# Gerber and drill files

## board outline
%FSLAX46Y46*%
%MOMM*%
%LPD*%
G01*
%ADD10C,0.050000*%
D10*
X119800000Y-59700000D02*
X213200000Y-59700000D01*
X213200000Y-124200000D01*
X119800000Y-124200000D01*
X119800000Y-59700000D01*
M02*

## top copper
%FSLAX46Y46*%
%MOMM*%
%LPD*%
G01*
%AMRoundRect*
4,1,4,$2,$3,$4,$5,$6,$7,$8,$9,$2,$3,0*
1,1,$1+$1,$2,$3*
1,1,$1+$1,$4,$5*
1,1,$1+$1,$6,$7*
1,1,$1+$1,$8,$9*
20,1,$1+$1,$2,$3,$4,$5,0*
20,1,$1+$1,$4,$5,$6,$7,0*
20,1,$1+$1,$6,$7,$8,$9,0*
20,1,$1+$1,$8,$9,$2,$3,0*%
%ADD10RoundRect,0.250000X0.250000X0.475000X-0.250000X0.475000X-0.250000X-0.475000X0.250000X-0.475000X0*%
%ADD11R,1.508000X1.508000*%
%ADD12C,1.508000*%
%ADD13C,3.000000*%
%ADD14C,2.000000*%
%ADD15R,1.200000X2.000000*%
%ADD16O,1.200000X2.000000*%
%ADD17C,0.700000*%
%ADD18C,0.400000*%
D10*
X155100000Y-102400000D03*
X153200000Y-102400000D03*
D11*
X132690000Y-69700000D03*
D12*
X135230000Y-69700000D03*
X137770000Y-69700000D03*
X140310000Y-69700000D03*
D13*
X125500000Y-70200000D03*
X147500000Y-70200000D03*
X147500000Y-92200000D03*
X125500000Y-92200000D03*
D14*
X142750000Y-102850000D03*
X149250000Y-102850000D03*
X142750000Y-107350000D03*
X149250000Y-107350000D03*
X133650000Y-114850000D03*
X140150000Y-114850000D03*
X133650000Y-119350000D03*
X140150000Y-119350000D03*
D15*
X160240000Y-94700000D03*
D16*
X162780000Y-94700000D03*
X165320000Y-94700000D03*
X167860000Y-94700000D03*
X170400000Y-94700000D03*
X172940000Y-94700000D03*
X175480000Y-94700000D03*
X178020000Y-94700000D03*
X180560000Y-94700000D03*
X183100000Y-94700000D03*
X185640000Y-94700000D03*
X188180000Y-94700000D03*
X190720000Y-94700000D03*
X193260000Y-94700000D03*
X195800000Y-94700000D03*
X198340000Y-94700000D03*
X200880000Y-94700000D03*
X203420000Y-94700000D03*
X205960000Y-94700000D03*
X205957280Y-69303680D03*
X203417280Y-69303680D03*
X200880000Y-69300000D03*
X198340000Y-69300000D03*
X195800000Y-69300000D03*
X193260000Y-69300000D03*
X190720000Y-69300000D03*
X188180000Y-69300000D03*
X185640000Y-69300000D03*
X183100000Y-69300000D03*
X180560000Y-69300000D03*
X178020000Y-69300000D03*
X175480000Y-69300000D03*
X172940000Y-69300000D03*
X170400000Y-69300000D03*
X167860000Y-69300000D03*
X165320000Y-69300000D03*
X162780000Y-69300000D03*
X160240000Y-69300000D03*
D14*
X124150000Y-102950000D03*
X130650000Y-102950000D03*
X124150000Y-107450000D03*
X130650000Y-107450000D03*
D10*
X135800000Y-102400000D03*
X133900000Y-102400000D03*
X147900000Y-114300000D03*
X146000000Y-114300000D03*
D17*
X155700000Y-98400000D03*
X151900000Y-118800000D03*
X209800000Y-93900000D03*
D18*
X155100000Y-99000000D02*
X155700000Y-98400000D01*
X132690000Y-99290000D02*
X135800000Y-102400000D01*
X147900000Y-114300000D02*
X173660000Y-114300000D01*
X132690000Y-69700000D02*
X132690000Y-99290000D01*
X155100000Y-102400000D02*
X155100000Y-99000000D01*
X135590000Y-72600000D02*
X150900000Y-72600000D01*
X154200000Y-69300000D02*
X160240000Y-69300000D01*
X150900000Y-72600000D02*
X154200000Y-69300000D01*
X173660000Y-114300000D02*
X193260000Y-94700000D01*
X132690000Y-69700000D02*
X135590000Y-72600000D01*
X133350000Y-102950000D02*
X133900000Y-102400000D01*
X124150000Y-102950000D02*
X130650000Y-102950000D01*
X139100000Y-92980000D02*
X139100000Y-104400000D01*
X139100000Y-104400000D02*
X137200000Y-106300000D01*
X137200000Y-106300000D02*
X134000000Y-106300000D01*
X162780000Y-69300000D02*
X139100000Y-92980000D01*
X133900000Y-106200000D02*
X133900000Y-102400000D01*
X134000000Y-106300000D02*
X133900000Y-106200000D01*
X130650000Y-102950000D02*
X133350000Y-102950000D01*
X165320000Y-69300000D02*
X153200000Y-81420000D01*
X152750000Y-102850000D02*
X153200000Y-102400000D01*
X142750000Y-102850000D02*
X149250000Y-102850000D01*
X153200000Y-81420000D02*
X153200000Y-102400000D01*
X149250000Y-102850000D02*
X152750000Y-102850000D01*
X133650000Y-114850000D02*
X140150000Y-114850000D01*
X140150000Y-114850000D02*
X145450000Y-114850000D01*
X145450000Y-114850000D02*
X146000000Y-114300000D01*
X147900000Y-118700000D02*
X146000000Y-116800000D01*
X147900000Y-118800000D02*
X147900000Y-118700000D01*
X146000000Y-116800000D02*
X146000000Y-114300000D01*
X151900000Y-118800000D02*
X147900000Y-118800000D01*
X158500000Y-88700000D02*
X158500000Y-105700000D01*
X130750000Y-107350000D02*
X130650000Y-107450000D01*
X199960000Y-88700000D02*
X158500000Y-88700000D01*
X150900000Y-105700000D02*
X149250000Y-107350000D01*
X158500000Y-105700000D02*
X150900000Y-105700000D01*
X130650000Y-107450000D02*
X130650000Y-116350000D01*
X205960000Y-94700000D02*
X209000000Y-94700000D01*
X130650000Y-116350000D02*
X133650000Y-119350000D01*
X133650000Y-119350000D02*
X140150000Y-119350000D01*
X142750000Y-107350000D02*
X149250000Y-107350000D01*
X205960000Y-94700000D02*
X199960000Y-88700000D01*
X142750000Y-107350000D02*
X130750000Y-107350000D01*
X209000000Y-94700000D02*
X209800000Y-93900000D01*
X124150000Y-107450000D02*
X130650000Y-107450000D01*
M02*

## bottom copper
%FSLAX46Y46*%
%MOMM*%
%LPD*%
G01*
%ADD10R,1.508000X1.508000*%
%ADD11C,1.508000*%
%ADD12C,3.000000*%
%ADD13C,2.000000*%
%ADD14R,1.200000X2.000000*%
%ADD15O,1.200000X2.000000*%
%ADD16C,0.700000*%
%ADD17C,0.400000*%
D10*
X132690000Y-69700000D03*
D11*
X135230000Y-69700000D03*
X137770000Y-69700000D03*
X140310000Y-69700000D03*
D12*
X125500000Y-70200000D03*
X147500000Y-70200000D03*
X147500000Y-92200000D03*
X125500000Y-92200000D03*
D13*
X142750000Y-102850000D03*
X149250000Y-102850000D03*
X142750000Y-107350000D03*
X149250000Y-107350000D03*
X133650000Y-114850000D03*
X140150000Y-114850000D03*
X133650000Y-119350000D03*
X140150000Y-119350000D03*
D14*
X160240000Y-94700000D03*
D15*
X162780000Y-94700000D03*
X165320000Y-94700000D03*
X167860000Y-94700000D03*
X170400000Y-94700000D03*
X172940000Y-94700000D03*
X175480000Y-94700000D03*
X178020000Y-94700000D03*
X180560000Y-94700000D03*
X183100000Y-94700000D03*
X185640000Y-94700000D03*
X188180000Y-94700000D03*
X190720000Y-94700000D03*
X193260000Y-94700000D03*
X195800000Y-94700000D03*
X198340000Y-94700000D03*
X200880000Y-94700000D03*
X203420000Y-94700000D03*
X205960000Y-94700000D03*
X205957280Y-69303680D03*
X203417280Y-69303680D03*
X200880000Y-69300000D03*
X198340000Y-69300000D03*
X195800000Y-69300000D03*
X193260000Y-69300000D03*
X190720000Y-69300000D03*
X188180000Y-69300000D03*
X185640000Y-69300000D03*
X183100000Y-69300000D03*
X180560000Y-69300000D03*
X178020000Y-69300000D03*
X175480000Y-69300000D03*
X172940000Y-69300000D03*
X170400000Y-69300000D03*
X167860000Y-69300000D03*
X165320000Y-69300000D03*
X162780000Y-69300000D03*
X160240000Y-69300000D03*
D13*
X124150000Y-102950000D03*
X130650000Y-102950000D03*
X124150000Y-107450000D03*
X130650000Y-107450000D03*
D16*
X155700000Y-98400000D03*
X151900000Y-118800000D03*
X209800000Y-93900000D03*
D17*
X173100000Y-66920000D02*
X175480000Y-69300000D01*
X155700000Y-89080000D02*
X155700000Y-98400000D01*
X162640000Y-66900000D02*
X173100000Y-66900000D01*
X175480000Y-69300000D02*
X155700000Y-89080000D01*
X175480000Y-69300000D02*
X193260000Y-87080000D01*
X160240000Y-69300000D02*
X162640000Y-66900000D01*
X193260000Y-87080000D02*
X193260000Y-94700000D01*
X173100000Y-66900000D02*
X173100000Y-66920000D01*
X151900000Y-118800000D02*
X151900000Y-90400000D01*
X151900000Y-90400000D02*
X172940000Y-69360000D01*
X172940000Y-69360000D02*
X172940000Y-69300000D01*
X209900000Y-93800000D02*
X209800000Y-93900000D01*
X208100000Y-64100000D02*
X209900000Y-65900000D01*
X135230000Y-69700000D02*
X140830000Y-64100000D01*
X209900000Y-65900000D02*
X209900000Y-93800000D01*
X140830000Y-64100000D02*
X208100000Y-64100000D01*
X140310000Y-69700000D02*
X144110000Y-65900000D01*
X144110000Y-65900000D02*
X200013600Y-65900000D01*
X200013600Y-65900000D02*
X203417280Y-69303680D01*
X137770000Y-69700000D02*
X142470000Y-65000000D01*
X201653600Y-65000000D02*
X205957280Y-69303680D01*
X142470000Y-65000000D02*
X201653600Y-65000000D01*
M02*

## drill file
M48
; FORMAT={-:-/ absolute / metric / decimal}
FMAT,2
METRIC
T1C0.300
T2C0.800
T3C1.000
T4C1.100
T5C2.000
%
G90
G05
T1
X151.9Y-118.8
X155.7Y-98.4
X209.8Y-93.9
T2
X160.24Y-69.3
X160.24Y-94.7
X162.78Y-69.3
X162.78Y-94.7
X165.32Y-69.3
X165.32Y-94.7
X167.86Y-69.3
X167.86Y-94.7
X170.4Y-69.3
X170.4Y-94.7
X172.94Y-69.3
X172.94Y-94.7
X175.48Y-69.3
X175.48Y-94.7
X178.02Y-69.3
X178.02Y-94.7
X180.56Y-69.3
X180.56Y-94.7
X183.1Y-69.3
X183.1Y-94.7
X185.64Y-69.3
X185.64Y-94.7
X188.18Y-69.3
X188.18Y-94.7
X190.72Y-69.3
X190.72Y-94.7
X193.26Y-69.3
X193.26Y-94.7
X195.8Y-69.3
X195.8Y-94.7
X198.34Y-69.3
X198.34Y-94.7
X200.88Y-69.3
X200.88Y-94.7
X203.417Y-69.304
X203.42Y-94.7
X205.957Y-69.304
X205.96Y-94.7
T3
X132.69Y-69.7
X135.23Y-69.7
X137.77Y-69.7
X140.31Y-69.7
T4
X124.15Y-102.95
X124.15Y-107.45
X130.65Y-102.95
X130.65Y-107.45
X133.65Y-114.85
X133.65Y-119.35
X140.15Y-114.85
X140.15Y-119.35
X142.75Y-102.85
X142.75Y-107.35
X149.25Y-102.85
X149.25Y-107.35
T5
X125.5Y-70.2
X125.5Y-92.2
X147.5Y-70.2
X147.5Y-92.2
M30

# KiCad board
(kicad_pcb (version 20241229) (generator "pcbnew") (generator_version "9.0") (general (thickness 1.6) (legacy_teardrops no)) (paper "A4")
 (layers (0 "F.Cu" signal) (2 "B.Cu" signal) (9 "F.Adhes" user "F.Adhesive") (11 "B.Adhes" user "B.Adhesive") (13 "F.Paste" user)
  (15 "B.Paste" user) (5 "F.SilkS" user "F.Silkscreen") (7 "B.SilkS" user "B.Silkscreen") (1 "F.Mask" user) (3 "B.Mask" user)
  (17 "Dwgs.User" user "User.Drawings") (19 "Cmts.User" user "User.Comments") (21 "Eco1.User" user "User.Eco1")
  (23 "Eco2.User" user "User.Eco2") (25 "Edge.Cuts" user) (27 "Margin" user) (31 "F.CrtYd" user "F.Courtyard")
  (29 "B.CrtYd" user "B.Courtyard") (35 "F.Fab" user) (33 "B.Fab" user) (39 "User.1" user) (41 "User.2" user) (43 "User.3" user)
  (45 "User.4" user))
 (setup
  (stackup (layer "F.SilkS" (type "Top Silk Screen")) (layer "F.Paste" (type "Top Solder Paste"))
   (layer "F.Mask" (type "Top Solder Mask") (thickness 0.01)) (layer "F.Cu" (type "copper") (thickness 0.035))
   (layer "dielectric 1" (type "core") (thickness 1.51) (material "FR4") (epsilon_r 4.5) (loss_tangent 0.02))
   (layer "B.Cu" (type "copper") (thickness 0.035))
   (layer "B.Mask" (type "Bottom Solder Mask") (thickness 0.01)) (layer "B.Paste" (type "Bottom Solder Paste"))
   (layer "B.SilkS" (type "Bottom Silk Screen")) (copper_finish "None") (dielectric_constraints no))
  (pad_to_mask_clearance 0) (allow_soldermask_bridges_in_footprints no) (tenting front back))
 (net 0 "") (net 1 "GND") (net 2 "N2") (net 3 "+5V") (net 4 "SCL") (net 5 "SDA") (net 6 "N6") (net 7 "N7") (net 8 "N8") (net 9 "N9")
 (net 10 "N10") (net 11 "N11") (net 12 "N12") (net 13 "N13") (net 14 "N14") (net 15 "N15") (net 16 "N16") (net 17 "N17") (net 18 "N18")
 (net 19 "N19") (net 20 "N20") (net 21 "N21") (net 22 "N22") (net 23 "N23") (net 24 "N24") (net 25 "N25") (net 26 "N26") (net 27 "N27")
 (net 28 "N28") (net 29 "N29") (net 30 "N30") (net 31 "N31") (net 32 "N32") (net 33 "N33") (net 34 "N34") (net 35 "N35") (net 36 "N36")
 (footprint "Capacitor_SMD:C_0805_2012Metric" (layer "F.Cu") (at 154.15 102.4 180)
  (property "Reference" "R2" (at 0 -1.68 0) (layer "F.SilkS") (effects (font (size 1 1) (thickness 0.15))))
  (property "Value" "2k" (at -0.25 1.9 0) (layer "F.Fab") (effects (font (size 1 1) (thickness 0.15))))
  (pad "1" smd roundrect (at -0.95 0 180) (size 1 1.45) (layers "F.Cu" "F.Mask" "F.Paste") (roundrect_rratio 0.25) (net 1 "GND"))
  (pad "2" smd roundrect (at 0.95 0 180) (size 1 1.45) (layers "F.Cu" "F.Mask" "F.Paste") (roundrect_rratio 0.25) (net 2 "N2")))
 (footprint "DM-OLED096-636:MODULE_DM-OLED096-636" (layer "F.Cu") (at 136.5 81.2)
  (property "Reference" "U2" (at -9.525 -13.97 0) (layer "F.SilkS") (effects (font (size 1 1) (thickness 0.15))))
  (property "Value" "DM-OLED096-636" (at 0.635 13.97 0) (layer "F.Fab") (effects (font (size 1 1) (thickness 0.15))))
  (pad "1" thru_hole rect (at -3.81 -11.5) (size 1.508 1.508) (drill 1) (layers "*.Cu" "*.Mask") (remove_unused_layers no) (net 1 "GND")
   (solder_mask_margin 0.102))
  (pad "2" thru_hole circle (at -1.27 -11.5) (size 1.508 1.508) (drill 1) (layers "*.Cu" "*.Mask") (remove_unused_layers no) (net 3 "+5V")
   (solder_mask_margin 0.102))
  (pad "3" thru_hole circle (at 1.27 -11.5) (size 1.508 1.508) (drill 1) (layers "*.Cu" "*.Mask") (remove_unused_layers no) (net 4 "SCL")
   (solder_mask_margin 0.102))
  (pad "4" thru_hole circle (at 3.81 -11.5) (size 1.508 1.508) (drill 1) (layers "*.Cu" "*.Mask") (remove_unused_layers no) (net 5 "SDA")
   (solder_mask_margin 0.102))
  (pad "S1" thru_hole circle (at -11 -11) (size 3 3) (drill 2) (layers "*.Cu" "*.Mask") (remove_unused_layers no) (solder_mask_margin 0.102))
  (pad "S2" thru_hole circle (at 11 -11) (size 3 3) (drill 2) (layers "*.Cu" "*.Mask") (remove_unused_layers no) (solder_mask_margin 0.102))
  (pad "S3" thru_hole circle (at 11 11) (size 3 3) (drill 2) (layers "*.Cu" "*.Mask") (remove_unused_layers no) (solder_mask_margin 0.102))
  (pad "S4" thru_hole circle (at -11 11) (size 3 3) (drill 2) (layers "*.Cu" "*.Mask") (remove_unused_layers no) (solder_mask_margin 0.102)))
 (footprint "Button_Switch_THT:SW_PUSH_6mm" (layer "F.Cu") (at 142.75 102.85)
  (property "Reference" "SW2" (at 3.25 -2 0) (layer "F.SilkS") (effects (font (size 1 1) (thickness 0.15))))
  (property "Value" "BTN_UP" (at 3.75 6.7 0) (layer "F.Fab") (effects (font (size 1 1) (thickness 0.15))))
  (pad "1" thru_hole circle (at 0 0 90) (size 2 2) (drill 1.1) (layers "*.Cu" "*.Mask") (remove_unused_layers no) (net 2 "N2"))
  (pad "1" thru_hole circle (at 6.5 0 90) (size 2 2) (drill 1.1) (layers "*.Cu" "*.Mask") (remove_unused_layers no) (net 2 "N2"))
  (pad "2" thru_hole circle (at 0 4.5 90) (size 2 2) (drill 1.1) (layers "*.Cu" "*.Mask") (remove_unused_layers no) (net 3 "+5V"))
  (pad "2" thru_hole circle (at 6.5 4.5 90) (size 2 2) (drill 1.1) (layers "*.Cu" "*.Mask") (remove_unused_layers no) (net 3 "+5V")))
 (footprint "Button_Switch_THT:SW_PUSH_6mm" (layer "F.Cu") (at 133.65 114.85)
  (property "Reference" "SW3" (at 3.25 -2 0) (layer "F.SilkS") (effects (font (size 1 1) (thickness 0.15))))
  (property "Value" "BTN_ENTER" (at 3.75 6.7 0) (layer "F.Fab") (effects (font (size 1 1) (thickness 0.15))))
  (pad "1" thru_hole circle (at 0 0 90) (size 2 2) (drill 1.1) (layers "*.Cu" "*.Mask") (remove_unused_layers no) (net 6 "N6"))
  (pad "1" thru_hole circle (at 6.5 0 90) (size 2 2) (drill 1.1) (layers "*.Cu" "*.Mask") (remove_unused_layers no) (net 6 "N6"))
  (pad "2" thru_hole circle (at 0 4.5 90) (size 2 2) (drill 1.1) (layers "*.Cu" "*.Mask") (remove_unused_layers no) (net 3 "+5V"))
  (pad "2" thru_hole circle (at 6.5 4.5 90) (size 2 2) (drill 1.1) (layers "*.Cu" "*.Mask") (remove_unused_layers no) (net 3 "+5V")))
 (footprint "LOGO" (layer "F.Cu") (at 189.2 112.5)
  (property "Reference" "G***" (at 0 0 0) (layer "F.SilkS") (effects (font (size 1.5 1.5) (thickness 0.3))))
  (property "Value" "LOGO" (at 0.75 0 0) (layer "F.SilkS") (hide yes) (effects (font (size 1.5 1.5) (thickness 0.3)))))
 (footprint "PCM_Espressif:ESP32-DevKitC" (layer "F.Cu") (at 160.24 94.7 90)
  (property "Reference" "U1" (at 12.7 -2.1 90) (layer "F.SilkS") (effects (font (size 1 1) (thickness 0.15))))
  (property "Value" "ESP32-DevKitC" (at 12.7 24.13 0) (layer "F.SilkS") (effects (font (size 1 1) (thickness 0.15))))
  (pad "1" thru_hole rect (at 0 0) (size 1.2 2) (drill 0.8) (layers "*.Cu" "*.Mask") (remove_unused_layers no) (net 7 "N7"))
  (pad "2" thru_hole oval (at 0 2.54) (size 1.2 2) (drill 0.8) (layers "*.Cu" "*.Mask") (remove_unused_layers no) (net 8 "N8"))
  (pad "3" thru_hole oval (at 0 5.08) (size 1.2 2) (drill 0.8) (layers "*.Cu" "*.Mask") (remove_unused_layers no) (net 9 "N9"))
  (pad "4" thru_hole oval (at 0 7.62) (size 1.2 2) (drill 0.8) (layers "*.Cu" "*.Mask") (remove_unused_layers no) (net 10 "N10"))
  (pad "5" thru_hole oval (at 0 10.16) (size 1.2 2) (drill 0.8) (layers "*.Cu" "*.Mask") (remove_unused_layers no) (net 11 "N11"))
  (pad "6" thru_hole oval (at 0 12.7) (size 1.2 2) (drill 0.8) (layers "*.Cu" "*.Mask") (remove_unused_layers no) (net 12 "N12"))
  (pad "7" thru_hole oval (at 0 15.24) (size 1.2 2) (drill 0.8) (layers "*.Cu" "*.Mask") (remove_unused_layers no) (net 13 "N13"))
  (pad "8" thru_hole oval (at 0 17.78) (size 1.2 2) (drill 0.8) (layers "*.Cu" "*.Mask") (remove_unused_layers no) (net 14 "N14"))
  (pad "9" thru_hole oval (at 0 20.32) (size 1.2 2) (drill 0.8) (layers "*.Cu" "*.Mask") (remove_unused_layers no) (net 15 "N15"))
  (pad "10" thru_hole oval (at 0 22.86) (size 1.2 2) (drill 0.8) (layers "*.Cu" "*.Mask") (remove_unused_layers no) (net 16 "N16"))
  (pad "11" thru_hole oval (at 0 25.4) (size 1.2 2) (drill 0.8) (layers "*.Cu" "*.Mask") (remove_unused_layers no) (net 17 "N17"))
  (pad "12" thru_hole oval (at 0 27.94) (size 1.2 2) (drill 0.8) (layers "*.Cu" "*.Mask") (remove_unused_layers no) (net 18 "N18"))
  (pad "13" thru_hole oval (at 0 30.48) (size 1.2 2) (drill 0.8) (layers "*.Cu" "*.Mask") (remove_unused_layers no) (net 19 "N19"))
  (pad "14" thru_hole oval (at 0 33.02) (size 1.2 2) (drill 0.8) (layers "*.Cu" "*.Mask") (remove_unused_layers no) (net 1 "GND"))
  (pad "15" thru_hole oval (at 0 35.56) (size 1.2 2) (drill 0.8) (layers "*.Cu" "*.Mask") (remove_unused_layers no) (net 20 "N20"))
  (pad "16" thru_hole oval (at 0 38.1) (size 1.2 2) (drill 0.8) (layers "*.Cu" "*.Mask") (remove_unused_layers no) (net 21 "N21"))
  (pad "17" thru_hole oval (at 0 40.64) (size 1.2 2) (drill 0.8) (layers "*.Cu" "*.Mask") (remove_unused_layers no) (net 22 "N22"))
  (pad "18" thru_hole oval (at 0 43.18) (size 1.2 2) (drill 0.8) (layers "*.Cu" "*.Mask") (remove_unused_layers no) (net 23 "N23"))
  (pad "19" thru_hole oval (at 0 45.72) (size 1.2 2) (drill 0.8) (layers "*.Cu" "*.Mask") (remove_unused_layers no) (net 3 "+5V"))
  (pad "20" thru_hole oval (at 25.39632 45.71728) (size 1.2 2) (drill 0.8) (layers "*.Cu" "*.Mask") (remove_unused_layers no) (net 4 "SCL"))
  (pad "21" thru_hole oval (at 25.39632 43.17728) (size 1.2 2) (drill 0.8) (layers "*.Cu" "*.Mask") (remove_unused_layers no) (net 5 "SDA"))
  (pad "22" thru_hole oval (at 25.4 40.64) (size 1.2 2) (drill 0.8) (layers "*.Cu" "*.Mask") (remove_unused_layers no) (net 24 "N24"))
  (pad "23" thru_hole oval (at 25.4 38.1) (size 1.2 2) (drill 0.8) (layers "*.Cu" "*.Mask") (remove_unused_layers no) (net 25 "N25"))
  (pad "24" thru_hole oval (at 25.4 35.56) (size 1.2 2) (drill 0.8) (layers "*.Cu" "*.Mask") (remove_unused_layers no) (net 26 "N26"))
  (pad "25" thru_hole oval (at 25.4 33.02) (size 1.2 2) (drill 0.8) (layers "*.Cu" "*.Mask") (remove_unused_layers no) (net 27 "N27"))
  (pad "26" thru_hole oval (at 25.4 30.48) (size 1.2 2) (drill 0.8) (layers "*.Cu" "*.Mask") (remove_unused_layers no) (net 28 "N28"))
  (pad "27" thru_hole oval (at 25.4 27.94) (size 1.2 2) (drill 0.8) (layers "*.Cu" "*.Mask") (remove_unused_layers no) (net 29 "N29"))
  (pad "28" thru_hole oval (at 25.4 25.4) (size 1.2 2) (drill 0.8) (layers "*.Cu" "*.Mask") (remove_unused_layers no) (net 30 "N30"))
  (pad "29" thru_hole oval (at 25.4 22.86) (size 1.2 2) (drill 0.8) (layers "*.Cu" "*.Mask") (remove_unused_layers no) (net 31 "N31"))
  (pad "30" thru_hole oval (at 25.4 20.32) (size 1.2 2) (drill 0.8) (layers "*.Cu" "*.Mask") (remove_unused_layers no) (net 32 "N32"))
  (pad "31" thru_hole oval (at 25.4 17.78) (size 1.2 2) (drill 0.8) (layers "*.Cu" "*.Mask") (remove_unused_layers no) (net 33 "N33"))
  (pad "32" thru_hole oval (at 25.4 15.24) (size 1.2 2) (drill 0.8) (layers "*.Cu" "*.Mask") (remove_unused_layers no) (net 1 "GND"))
  (pad "33" thru_hole oval (at 25.4 12.7) (size 1.2 2) (drill 0.8) (layers "*.Cu" "*.Mask") (remove_unused_layers no) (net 6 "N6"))
  (pad "34" thru_hole oval (at 25.4 10.16) (size 1.2 2) (drill 0.8) (layers "*.Cu" "*.Mask") (remove_unused_layers no) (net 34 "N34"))
  (pad "35" thru_hole oval (at 25.4 7.62) (size 1.2 2) (drill 0.8) (layers "*.Cu" "*.Mask") (remove_unused_layers no) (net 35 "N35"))
  (pad "36" thru_hole oval (at 25.4 5.08) (size 1.2 2) (drill 0.8) (layers "*.Cu" "*.Mask") (remove_unused_layers no) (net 2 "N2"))
  (pad "37" thru_hole oval (at 25.4 2.54) (size 1.2 2) (drill 0.8) (layers "*.Cu" "*.Mask") (remove_unused_layers no) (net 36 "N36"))
  (pad "38" thru_hole oval (at 25.4 0) (size 1.2 2) (drill 0.8) (layers "*.Cu" "*.Mask") (remove_unused_layers no) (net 1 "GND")))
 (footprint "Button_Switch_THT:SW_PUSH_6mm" (layer "F.Cu") (at 124.15 102.95)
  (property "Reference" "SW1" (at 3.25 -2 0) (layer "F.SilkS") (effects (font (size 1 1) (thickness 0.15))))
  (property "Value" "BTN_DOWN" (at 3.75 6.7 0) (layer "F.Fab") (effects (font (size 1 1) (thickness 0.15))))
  (pad "1" thru_hole circle (at 0 0 90) (size 2 2) (drill 1.1) (layers "*.Cu" "*.Mask") (remove_unused_layers no) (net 36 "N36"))
  (pad "1" thru_hole circle (at 6.5 0 90) (size 2 2) (drill 1.1) (layers "*.Cu" "*.Mask") (remove_unused_layers no) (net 36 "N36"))
  (pad "2" thru_hole circle (at 0 4.5 90) (size 2 2) (drill 1.1) (layers "*.Cu" "*.Mask") (remove_unused_layers no) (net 3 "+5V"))
  (pad "2" thru_hole circle (at 6.5 4.5 90) (size 2 2) (drill 1.1) (layers "*.Cu" "*.Mask") (remove_unused_layers no) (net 3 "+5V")))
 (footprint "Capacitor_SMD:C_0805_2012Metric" (layer "F.Cu") (at 134.85 102.4 180)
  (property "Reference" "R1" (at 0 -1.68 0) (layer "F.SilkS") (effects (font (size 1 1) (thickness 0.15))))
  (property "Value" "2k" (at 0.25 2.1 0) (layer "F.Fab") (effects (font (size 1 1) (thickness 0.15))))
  (pad "1" smd roundrect (at -0.95 0 180) (size 1 1.45) (layers "F.Cu" "F.Mask" "F.Paste") (roundrect_rratio 0.25) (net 1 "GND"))
  (pad "2" smd roundrect (at 0.95 0 180) (size 1 1.45) (layers "F.Cu" "F.Mask" "F.Paste") (roundrect_rratio 0.25) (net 36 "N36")))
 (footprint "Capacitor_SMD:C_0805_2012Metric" (layer "F.Cu") (at 146.95 114.3 180)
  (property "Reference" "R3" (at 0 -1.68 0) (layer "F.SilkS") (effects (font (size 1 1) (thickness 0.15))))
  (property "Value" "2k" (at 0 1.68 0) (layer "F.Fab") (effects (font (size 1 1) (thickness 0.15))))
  (pad "1" smd roundrect (at -0.95 0 180) (size 1 1.45) (layers "F.Cu" "F.Mask" "F.Paste") (roundrect_rratio 0.25) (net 1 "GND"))
  (pad "2" smd roundrect (at 0.95 0 180) (size 1 1.45) (layers "F.Cu" "F.Mask" "F.Paste") (roundrect_rratio 0.25) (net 6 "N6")))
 (gr_rect (start 119.8 59.7) (end 213.2 124.2) (stroke (width 0.05) (type default)) (fill no) (layer "Edge.Cuts"))
 (segment (start 155.1 99) (end 155.7 98.4) (width 0.4) (layer "F.Cu") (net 1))
 (segment (start 132.69 99.29) (end 135.8 102.4) (width 0.4) (layer "F.Cu") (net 1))
 (segment (start 147.9 114.3) (end 173.66 114.3) (width 0.4) (layer "F.Cu") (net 1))
 (segment (start 132.69 69.7) (end 132.69 99.29) (width 0.4) (layer "F.Cu") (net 1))
 (segment (start 155.1 102.4) (end 155.1 99) (width 0.4) (layer "F.Cu") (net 1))
 (segment (start 135.59 72.6) (end 150.9 72.6) (width 0.4) (layer "F.Cu") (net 1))
 (segment (start 154.2 69.3) (end 160.24 69.3) (width 0.4) (layer "F.Cu") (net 1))
 (segment (start 150.9 72.6) (end 154.2 69.3) (width 0.4) (layer "F.Cu") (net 1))
 (segment (start 173.66 114.3) (end 193.26 94.7) (width 0.4) (layer "F.Cu") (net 1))
 (segment (start 132.69 69.7) (end 135.59 72.6) (width 0.4) (layer "F.Cu") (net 1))
 (via (at 155.7 98.4) (size 0.7) (drill 0.3) (layers "F.Cu" "B.Cu") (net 1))
 (segment (start 173.1 66.92) (end 175.48 69.3) (width 0.4) (layer "B.Cu") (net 1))
 (segment (start 155.7 89.08) (end 155.7 98.4) (width 0.4) (layer "B.Cu") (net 1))
 (segment (start 162.64 66.9) (end 173.1 66.9) (width 0.4) (layer "B.Cu") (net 1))
 (segment (start 175.48 69.3) (end 155.7 89.08) (width 0.4) (layer "B.Cu") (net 1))
 (segment (start 175.48 69.3) (end 193.26 87.08) (width 0.4) (layer "B.Cu") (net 1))
 (segment (start 160.24 69.3) (end 162.64 66.9) (width 0.4) (layer "B.Cu") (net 1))
 (segment (start 193.26 87.08) (end 193.26 94.7) (width 0.4) (layer "B.Cu") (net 1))
 (segment (start 173.1 66.9) (end 173.1 66.92) (width 0.4) (layer "B.Cu") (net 1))
 (segment (start 133.35 102.95) (end 133.9 102.4) (width 0.4) (layer "F.Cu") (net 36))
 (segment (start 124.15 102.95) (end 130.65 102.95) (width 0.4) (layer "F.Cu") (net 36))
 (segment (start 139.1 92.98) (end 139.1 104.4) (width 0.4) (layer "F.Cu") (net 36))
 (segment (start 139.1 104.4) (end 137.2 106.3) (width 0.4) (layer "F.Cu") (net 36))
 (segment (start 137.2 106.3) (end 134 106.3) (width 0.4) (layer "F.Cu") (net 36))
 (segment (start 162.78 69.3) (end 139.1 92.98) (width 0.4) (layer "F.Cu") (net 36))
 (segment (start 133.9 106.2) (end 133.9 102.4) (width 0.4) (layer "F.Cu") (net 36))
 (segment (start 134 106.3) (end 133.9 106.2) (width 0.4) (layer "F.Cu") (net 36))
 (segment (start 130.65 102.95) (end 133.35 102.95) (width 0.4) (layer "F.Cu") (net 36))
 (segment (start 165.32 69.3) (end 153.2 81.42) (width 0.4) (layer "F.Cu") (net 2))
 (segment (start 152.75 102.85) (end 153.2 102.4) (width 0.4) (layer "F.Cu") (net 2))
 (segment (start 142.75 102.85) (end 149.25 102.85) (width 0.4) (layer "F.Cu") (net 2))
 (segment (start 153.2 81.42) (end 153.2 102.4) (width 0.4) (layer "F.Cu") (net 2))
 (segment (start 149.25 102.85) (end 152.75 102.85) (width 0.4) (layer "F.Cu") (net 2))
 (segment (start 133.65 114.85) (end 140.15 114.85) (width 0.4) (layer "F.Cu") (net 6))
 (segment (start 140.15 114.85) (end 145.45 114.85) (width 0.4) (layer "F.Cu") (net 6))
 (segment (start 145.45 114.85) (end 146 114.3) (width 0.4) (layer "F.Cu") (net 6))
 (segment (start 147.9 118.7) (end 146 116.8) (width 0.4) (layer "F.Cu") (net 6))
 (segment (start 147.9 118.8) (end 147.9 118.7) (width 0.4) (layer "F.Cu") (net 6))
 (segment (start 146 116.8) (end 146 114.3) (width 0.4) (layer "F.Cu") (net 6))
 (segment (start 151.9 118.8) (end 147.9 118.8) (width 0.4) (layer "F.Cu") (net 6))
 (via (at 151.9 118.8) (size 0.7) (drill 0.3) (layers "F.Cu" "B.Cu") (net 6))
 (segment (start 151.9 118.8) (end 151.9 90.4) (width 0.4) (layer "B.Cu") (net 6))
 (segment (start 151.9 90.4) (end 172.94 69.36) (width 0.4) (layer "B.Cu") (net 6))
 (segment (start 172.94 69.36) (end 172.94 69.3) (width 0.4) (layer "B.Cu") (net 6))
 (segment (start 158.5 88.7) (end 158.5 105.7) (width 0.4) (layer "F.Cu") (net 3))
 (segment (start 130.75 107.35) (end 130.65 107.45) (width 0.4) (layer "F.Cu") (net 3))
 (segment (start 199.96 88.7) (end 158.5 88.7) (width 0.4) (layer "F.Cu") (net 3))
 (segment (start 150.9 105.7) (end 149.25 107.35) (width 0.4) (layer "F.Cu") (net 3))
 (segment (start 158.5 105.7) (end 150.9 105.7) (width 0.4) (layer "F.Cu") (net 3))
 (segment (start 130.65 107.45) (end 130.65 116.35) (width 0.4) (layer "F.Cu") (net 3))
 (segment (start 205.96 94.7) (end 209 94.7) (width 0.4) (layer "F.Cu") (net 3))
 (segment (start 130.65 116.35) (end 133.65 119.35) (width 0.4) (layer "F.Cu") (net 3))
 (segment (start 133.65 119.35) (end 140.15 119.35) (width 0.4) (layer "F.Cu") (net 3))
 (segment (start 142.75 107.35) (end 149.25 107.35) (width 0.4) (layer "F.Cu") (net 3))
 (segment (start 205.96 94.7) (end 199.96 88.7) (width 0.4) (layer "F.Cu") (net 3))
 (segment (start 142.75 107.35) (end 130.75 107.35) (width 0.4) (layer "F.Cu") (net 3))
 (segment (start 209 94.7) (end 209.8 93.9) (width 0.4) (layer "F.Cu") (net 3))
 (segment (start 124.15 107.45) (end 130.65 107.45) (width 0.4) (layer "F.Cu") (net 3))
 (via (at 209.8 93.9) (size 0.7) (drill 0.3) (layers "F.Cu" "B.Cu") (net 3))
 (segment (start 209.9 93.8) (end 209.8 93.9) (width 0.4) (layer "B.Cu") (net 3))
 (segment (start 208.1 64.1) (end 209.9 65.9) (width 0.4) (layer "B.Cu") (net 3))
 (segment (start 135.23 69.7) (end 140.83 64.1) (width 0.4) (layer "B.Cu") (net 3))
 (segment (start 209.9 65.9) (end 209.9 93.8) (width 0.4) (layer "B.Cu") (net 3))
 (segment (start 140.83 64.1) (end 208.1 64.1) (width 0.4) (layer "B.Cu") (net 3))
 (segment (start 140.31 69.7) (end 144.11 65.9) (width 0.4) (layer "B.Cu") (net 5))
 (segment (start 144.11 65.9) (end 200.0136 65.9) (width 0.4) (layer "B.Cu") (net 5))
 (segment (start 200.0136 65.9) (end 203.41728 69.30368) (width 0.4) (layer "B.Cu") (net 5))
 (segment (start 137.77 69.7) (end 142.47 65) (width 0.4) (layer "B.Cu") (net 4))
 (segment (start 201.6536 65) (end 205.95728 69.30368) (width 0.4) (layer "B.Cu") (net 4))
 (segment (start 142.47 65) (end 201.6536 65) (width 0.4) (layer "B.Cu") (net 4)))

